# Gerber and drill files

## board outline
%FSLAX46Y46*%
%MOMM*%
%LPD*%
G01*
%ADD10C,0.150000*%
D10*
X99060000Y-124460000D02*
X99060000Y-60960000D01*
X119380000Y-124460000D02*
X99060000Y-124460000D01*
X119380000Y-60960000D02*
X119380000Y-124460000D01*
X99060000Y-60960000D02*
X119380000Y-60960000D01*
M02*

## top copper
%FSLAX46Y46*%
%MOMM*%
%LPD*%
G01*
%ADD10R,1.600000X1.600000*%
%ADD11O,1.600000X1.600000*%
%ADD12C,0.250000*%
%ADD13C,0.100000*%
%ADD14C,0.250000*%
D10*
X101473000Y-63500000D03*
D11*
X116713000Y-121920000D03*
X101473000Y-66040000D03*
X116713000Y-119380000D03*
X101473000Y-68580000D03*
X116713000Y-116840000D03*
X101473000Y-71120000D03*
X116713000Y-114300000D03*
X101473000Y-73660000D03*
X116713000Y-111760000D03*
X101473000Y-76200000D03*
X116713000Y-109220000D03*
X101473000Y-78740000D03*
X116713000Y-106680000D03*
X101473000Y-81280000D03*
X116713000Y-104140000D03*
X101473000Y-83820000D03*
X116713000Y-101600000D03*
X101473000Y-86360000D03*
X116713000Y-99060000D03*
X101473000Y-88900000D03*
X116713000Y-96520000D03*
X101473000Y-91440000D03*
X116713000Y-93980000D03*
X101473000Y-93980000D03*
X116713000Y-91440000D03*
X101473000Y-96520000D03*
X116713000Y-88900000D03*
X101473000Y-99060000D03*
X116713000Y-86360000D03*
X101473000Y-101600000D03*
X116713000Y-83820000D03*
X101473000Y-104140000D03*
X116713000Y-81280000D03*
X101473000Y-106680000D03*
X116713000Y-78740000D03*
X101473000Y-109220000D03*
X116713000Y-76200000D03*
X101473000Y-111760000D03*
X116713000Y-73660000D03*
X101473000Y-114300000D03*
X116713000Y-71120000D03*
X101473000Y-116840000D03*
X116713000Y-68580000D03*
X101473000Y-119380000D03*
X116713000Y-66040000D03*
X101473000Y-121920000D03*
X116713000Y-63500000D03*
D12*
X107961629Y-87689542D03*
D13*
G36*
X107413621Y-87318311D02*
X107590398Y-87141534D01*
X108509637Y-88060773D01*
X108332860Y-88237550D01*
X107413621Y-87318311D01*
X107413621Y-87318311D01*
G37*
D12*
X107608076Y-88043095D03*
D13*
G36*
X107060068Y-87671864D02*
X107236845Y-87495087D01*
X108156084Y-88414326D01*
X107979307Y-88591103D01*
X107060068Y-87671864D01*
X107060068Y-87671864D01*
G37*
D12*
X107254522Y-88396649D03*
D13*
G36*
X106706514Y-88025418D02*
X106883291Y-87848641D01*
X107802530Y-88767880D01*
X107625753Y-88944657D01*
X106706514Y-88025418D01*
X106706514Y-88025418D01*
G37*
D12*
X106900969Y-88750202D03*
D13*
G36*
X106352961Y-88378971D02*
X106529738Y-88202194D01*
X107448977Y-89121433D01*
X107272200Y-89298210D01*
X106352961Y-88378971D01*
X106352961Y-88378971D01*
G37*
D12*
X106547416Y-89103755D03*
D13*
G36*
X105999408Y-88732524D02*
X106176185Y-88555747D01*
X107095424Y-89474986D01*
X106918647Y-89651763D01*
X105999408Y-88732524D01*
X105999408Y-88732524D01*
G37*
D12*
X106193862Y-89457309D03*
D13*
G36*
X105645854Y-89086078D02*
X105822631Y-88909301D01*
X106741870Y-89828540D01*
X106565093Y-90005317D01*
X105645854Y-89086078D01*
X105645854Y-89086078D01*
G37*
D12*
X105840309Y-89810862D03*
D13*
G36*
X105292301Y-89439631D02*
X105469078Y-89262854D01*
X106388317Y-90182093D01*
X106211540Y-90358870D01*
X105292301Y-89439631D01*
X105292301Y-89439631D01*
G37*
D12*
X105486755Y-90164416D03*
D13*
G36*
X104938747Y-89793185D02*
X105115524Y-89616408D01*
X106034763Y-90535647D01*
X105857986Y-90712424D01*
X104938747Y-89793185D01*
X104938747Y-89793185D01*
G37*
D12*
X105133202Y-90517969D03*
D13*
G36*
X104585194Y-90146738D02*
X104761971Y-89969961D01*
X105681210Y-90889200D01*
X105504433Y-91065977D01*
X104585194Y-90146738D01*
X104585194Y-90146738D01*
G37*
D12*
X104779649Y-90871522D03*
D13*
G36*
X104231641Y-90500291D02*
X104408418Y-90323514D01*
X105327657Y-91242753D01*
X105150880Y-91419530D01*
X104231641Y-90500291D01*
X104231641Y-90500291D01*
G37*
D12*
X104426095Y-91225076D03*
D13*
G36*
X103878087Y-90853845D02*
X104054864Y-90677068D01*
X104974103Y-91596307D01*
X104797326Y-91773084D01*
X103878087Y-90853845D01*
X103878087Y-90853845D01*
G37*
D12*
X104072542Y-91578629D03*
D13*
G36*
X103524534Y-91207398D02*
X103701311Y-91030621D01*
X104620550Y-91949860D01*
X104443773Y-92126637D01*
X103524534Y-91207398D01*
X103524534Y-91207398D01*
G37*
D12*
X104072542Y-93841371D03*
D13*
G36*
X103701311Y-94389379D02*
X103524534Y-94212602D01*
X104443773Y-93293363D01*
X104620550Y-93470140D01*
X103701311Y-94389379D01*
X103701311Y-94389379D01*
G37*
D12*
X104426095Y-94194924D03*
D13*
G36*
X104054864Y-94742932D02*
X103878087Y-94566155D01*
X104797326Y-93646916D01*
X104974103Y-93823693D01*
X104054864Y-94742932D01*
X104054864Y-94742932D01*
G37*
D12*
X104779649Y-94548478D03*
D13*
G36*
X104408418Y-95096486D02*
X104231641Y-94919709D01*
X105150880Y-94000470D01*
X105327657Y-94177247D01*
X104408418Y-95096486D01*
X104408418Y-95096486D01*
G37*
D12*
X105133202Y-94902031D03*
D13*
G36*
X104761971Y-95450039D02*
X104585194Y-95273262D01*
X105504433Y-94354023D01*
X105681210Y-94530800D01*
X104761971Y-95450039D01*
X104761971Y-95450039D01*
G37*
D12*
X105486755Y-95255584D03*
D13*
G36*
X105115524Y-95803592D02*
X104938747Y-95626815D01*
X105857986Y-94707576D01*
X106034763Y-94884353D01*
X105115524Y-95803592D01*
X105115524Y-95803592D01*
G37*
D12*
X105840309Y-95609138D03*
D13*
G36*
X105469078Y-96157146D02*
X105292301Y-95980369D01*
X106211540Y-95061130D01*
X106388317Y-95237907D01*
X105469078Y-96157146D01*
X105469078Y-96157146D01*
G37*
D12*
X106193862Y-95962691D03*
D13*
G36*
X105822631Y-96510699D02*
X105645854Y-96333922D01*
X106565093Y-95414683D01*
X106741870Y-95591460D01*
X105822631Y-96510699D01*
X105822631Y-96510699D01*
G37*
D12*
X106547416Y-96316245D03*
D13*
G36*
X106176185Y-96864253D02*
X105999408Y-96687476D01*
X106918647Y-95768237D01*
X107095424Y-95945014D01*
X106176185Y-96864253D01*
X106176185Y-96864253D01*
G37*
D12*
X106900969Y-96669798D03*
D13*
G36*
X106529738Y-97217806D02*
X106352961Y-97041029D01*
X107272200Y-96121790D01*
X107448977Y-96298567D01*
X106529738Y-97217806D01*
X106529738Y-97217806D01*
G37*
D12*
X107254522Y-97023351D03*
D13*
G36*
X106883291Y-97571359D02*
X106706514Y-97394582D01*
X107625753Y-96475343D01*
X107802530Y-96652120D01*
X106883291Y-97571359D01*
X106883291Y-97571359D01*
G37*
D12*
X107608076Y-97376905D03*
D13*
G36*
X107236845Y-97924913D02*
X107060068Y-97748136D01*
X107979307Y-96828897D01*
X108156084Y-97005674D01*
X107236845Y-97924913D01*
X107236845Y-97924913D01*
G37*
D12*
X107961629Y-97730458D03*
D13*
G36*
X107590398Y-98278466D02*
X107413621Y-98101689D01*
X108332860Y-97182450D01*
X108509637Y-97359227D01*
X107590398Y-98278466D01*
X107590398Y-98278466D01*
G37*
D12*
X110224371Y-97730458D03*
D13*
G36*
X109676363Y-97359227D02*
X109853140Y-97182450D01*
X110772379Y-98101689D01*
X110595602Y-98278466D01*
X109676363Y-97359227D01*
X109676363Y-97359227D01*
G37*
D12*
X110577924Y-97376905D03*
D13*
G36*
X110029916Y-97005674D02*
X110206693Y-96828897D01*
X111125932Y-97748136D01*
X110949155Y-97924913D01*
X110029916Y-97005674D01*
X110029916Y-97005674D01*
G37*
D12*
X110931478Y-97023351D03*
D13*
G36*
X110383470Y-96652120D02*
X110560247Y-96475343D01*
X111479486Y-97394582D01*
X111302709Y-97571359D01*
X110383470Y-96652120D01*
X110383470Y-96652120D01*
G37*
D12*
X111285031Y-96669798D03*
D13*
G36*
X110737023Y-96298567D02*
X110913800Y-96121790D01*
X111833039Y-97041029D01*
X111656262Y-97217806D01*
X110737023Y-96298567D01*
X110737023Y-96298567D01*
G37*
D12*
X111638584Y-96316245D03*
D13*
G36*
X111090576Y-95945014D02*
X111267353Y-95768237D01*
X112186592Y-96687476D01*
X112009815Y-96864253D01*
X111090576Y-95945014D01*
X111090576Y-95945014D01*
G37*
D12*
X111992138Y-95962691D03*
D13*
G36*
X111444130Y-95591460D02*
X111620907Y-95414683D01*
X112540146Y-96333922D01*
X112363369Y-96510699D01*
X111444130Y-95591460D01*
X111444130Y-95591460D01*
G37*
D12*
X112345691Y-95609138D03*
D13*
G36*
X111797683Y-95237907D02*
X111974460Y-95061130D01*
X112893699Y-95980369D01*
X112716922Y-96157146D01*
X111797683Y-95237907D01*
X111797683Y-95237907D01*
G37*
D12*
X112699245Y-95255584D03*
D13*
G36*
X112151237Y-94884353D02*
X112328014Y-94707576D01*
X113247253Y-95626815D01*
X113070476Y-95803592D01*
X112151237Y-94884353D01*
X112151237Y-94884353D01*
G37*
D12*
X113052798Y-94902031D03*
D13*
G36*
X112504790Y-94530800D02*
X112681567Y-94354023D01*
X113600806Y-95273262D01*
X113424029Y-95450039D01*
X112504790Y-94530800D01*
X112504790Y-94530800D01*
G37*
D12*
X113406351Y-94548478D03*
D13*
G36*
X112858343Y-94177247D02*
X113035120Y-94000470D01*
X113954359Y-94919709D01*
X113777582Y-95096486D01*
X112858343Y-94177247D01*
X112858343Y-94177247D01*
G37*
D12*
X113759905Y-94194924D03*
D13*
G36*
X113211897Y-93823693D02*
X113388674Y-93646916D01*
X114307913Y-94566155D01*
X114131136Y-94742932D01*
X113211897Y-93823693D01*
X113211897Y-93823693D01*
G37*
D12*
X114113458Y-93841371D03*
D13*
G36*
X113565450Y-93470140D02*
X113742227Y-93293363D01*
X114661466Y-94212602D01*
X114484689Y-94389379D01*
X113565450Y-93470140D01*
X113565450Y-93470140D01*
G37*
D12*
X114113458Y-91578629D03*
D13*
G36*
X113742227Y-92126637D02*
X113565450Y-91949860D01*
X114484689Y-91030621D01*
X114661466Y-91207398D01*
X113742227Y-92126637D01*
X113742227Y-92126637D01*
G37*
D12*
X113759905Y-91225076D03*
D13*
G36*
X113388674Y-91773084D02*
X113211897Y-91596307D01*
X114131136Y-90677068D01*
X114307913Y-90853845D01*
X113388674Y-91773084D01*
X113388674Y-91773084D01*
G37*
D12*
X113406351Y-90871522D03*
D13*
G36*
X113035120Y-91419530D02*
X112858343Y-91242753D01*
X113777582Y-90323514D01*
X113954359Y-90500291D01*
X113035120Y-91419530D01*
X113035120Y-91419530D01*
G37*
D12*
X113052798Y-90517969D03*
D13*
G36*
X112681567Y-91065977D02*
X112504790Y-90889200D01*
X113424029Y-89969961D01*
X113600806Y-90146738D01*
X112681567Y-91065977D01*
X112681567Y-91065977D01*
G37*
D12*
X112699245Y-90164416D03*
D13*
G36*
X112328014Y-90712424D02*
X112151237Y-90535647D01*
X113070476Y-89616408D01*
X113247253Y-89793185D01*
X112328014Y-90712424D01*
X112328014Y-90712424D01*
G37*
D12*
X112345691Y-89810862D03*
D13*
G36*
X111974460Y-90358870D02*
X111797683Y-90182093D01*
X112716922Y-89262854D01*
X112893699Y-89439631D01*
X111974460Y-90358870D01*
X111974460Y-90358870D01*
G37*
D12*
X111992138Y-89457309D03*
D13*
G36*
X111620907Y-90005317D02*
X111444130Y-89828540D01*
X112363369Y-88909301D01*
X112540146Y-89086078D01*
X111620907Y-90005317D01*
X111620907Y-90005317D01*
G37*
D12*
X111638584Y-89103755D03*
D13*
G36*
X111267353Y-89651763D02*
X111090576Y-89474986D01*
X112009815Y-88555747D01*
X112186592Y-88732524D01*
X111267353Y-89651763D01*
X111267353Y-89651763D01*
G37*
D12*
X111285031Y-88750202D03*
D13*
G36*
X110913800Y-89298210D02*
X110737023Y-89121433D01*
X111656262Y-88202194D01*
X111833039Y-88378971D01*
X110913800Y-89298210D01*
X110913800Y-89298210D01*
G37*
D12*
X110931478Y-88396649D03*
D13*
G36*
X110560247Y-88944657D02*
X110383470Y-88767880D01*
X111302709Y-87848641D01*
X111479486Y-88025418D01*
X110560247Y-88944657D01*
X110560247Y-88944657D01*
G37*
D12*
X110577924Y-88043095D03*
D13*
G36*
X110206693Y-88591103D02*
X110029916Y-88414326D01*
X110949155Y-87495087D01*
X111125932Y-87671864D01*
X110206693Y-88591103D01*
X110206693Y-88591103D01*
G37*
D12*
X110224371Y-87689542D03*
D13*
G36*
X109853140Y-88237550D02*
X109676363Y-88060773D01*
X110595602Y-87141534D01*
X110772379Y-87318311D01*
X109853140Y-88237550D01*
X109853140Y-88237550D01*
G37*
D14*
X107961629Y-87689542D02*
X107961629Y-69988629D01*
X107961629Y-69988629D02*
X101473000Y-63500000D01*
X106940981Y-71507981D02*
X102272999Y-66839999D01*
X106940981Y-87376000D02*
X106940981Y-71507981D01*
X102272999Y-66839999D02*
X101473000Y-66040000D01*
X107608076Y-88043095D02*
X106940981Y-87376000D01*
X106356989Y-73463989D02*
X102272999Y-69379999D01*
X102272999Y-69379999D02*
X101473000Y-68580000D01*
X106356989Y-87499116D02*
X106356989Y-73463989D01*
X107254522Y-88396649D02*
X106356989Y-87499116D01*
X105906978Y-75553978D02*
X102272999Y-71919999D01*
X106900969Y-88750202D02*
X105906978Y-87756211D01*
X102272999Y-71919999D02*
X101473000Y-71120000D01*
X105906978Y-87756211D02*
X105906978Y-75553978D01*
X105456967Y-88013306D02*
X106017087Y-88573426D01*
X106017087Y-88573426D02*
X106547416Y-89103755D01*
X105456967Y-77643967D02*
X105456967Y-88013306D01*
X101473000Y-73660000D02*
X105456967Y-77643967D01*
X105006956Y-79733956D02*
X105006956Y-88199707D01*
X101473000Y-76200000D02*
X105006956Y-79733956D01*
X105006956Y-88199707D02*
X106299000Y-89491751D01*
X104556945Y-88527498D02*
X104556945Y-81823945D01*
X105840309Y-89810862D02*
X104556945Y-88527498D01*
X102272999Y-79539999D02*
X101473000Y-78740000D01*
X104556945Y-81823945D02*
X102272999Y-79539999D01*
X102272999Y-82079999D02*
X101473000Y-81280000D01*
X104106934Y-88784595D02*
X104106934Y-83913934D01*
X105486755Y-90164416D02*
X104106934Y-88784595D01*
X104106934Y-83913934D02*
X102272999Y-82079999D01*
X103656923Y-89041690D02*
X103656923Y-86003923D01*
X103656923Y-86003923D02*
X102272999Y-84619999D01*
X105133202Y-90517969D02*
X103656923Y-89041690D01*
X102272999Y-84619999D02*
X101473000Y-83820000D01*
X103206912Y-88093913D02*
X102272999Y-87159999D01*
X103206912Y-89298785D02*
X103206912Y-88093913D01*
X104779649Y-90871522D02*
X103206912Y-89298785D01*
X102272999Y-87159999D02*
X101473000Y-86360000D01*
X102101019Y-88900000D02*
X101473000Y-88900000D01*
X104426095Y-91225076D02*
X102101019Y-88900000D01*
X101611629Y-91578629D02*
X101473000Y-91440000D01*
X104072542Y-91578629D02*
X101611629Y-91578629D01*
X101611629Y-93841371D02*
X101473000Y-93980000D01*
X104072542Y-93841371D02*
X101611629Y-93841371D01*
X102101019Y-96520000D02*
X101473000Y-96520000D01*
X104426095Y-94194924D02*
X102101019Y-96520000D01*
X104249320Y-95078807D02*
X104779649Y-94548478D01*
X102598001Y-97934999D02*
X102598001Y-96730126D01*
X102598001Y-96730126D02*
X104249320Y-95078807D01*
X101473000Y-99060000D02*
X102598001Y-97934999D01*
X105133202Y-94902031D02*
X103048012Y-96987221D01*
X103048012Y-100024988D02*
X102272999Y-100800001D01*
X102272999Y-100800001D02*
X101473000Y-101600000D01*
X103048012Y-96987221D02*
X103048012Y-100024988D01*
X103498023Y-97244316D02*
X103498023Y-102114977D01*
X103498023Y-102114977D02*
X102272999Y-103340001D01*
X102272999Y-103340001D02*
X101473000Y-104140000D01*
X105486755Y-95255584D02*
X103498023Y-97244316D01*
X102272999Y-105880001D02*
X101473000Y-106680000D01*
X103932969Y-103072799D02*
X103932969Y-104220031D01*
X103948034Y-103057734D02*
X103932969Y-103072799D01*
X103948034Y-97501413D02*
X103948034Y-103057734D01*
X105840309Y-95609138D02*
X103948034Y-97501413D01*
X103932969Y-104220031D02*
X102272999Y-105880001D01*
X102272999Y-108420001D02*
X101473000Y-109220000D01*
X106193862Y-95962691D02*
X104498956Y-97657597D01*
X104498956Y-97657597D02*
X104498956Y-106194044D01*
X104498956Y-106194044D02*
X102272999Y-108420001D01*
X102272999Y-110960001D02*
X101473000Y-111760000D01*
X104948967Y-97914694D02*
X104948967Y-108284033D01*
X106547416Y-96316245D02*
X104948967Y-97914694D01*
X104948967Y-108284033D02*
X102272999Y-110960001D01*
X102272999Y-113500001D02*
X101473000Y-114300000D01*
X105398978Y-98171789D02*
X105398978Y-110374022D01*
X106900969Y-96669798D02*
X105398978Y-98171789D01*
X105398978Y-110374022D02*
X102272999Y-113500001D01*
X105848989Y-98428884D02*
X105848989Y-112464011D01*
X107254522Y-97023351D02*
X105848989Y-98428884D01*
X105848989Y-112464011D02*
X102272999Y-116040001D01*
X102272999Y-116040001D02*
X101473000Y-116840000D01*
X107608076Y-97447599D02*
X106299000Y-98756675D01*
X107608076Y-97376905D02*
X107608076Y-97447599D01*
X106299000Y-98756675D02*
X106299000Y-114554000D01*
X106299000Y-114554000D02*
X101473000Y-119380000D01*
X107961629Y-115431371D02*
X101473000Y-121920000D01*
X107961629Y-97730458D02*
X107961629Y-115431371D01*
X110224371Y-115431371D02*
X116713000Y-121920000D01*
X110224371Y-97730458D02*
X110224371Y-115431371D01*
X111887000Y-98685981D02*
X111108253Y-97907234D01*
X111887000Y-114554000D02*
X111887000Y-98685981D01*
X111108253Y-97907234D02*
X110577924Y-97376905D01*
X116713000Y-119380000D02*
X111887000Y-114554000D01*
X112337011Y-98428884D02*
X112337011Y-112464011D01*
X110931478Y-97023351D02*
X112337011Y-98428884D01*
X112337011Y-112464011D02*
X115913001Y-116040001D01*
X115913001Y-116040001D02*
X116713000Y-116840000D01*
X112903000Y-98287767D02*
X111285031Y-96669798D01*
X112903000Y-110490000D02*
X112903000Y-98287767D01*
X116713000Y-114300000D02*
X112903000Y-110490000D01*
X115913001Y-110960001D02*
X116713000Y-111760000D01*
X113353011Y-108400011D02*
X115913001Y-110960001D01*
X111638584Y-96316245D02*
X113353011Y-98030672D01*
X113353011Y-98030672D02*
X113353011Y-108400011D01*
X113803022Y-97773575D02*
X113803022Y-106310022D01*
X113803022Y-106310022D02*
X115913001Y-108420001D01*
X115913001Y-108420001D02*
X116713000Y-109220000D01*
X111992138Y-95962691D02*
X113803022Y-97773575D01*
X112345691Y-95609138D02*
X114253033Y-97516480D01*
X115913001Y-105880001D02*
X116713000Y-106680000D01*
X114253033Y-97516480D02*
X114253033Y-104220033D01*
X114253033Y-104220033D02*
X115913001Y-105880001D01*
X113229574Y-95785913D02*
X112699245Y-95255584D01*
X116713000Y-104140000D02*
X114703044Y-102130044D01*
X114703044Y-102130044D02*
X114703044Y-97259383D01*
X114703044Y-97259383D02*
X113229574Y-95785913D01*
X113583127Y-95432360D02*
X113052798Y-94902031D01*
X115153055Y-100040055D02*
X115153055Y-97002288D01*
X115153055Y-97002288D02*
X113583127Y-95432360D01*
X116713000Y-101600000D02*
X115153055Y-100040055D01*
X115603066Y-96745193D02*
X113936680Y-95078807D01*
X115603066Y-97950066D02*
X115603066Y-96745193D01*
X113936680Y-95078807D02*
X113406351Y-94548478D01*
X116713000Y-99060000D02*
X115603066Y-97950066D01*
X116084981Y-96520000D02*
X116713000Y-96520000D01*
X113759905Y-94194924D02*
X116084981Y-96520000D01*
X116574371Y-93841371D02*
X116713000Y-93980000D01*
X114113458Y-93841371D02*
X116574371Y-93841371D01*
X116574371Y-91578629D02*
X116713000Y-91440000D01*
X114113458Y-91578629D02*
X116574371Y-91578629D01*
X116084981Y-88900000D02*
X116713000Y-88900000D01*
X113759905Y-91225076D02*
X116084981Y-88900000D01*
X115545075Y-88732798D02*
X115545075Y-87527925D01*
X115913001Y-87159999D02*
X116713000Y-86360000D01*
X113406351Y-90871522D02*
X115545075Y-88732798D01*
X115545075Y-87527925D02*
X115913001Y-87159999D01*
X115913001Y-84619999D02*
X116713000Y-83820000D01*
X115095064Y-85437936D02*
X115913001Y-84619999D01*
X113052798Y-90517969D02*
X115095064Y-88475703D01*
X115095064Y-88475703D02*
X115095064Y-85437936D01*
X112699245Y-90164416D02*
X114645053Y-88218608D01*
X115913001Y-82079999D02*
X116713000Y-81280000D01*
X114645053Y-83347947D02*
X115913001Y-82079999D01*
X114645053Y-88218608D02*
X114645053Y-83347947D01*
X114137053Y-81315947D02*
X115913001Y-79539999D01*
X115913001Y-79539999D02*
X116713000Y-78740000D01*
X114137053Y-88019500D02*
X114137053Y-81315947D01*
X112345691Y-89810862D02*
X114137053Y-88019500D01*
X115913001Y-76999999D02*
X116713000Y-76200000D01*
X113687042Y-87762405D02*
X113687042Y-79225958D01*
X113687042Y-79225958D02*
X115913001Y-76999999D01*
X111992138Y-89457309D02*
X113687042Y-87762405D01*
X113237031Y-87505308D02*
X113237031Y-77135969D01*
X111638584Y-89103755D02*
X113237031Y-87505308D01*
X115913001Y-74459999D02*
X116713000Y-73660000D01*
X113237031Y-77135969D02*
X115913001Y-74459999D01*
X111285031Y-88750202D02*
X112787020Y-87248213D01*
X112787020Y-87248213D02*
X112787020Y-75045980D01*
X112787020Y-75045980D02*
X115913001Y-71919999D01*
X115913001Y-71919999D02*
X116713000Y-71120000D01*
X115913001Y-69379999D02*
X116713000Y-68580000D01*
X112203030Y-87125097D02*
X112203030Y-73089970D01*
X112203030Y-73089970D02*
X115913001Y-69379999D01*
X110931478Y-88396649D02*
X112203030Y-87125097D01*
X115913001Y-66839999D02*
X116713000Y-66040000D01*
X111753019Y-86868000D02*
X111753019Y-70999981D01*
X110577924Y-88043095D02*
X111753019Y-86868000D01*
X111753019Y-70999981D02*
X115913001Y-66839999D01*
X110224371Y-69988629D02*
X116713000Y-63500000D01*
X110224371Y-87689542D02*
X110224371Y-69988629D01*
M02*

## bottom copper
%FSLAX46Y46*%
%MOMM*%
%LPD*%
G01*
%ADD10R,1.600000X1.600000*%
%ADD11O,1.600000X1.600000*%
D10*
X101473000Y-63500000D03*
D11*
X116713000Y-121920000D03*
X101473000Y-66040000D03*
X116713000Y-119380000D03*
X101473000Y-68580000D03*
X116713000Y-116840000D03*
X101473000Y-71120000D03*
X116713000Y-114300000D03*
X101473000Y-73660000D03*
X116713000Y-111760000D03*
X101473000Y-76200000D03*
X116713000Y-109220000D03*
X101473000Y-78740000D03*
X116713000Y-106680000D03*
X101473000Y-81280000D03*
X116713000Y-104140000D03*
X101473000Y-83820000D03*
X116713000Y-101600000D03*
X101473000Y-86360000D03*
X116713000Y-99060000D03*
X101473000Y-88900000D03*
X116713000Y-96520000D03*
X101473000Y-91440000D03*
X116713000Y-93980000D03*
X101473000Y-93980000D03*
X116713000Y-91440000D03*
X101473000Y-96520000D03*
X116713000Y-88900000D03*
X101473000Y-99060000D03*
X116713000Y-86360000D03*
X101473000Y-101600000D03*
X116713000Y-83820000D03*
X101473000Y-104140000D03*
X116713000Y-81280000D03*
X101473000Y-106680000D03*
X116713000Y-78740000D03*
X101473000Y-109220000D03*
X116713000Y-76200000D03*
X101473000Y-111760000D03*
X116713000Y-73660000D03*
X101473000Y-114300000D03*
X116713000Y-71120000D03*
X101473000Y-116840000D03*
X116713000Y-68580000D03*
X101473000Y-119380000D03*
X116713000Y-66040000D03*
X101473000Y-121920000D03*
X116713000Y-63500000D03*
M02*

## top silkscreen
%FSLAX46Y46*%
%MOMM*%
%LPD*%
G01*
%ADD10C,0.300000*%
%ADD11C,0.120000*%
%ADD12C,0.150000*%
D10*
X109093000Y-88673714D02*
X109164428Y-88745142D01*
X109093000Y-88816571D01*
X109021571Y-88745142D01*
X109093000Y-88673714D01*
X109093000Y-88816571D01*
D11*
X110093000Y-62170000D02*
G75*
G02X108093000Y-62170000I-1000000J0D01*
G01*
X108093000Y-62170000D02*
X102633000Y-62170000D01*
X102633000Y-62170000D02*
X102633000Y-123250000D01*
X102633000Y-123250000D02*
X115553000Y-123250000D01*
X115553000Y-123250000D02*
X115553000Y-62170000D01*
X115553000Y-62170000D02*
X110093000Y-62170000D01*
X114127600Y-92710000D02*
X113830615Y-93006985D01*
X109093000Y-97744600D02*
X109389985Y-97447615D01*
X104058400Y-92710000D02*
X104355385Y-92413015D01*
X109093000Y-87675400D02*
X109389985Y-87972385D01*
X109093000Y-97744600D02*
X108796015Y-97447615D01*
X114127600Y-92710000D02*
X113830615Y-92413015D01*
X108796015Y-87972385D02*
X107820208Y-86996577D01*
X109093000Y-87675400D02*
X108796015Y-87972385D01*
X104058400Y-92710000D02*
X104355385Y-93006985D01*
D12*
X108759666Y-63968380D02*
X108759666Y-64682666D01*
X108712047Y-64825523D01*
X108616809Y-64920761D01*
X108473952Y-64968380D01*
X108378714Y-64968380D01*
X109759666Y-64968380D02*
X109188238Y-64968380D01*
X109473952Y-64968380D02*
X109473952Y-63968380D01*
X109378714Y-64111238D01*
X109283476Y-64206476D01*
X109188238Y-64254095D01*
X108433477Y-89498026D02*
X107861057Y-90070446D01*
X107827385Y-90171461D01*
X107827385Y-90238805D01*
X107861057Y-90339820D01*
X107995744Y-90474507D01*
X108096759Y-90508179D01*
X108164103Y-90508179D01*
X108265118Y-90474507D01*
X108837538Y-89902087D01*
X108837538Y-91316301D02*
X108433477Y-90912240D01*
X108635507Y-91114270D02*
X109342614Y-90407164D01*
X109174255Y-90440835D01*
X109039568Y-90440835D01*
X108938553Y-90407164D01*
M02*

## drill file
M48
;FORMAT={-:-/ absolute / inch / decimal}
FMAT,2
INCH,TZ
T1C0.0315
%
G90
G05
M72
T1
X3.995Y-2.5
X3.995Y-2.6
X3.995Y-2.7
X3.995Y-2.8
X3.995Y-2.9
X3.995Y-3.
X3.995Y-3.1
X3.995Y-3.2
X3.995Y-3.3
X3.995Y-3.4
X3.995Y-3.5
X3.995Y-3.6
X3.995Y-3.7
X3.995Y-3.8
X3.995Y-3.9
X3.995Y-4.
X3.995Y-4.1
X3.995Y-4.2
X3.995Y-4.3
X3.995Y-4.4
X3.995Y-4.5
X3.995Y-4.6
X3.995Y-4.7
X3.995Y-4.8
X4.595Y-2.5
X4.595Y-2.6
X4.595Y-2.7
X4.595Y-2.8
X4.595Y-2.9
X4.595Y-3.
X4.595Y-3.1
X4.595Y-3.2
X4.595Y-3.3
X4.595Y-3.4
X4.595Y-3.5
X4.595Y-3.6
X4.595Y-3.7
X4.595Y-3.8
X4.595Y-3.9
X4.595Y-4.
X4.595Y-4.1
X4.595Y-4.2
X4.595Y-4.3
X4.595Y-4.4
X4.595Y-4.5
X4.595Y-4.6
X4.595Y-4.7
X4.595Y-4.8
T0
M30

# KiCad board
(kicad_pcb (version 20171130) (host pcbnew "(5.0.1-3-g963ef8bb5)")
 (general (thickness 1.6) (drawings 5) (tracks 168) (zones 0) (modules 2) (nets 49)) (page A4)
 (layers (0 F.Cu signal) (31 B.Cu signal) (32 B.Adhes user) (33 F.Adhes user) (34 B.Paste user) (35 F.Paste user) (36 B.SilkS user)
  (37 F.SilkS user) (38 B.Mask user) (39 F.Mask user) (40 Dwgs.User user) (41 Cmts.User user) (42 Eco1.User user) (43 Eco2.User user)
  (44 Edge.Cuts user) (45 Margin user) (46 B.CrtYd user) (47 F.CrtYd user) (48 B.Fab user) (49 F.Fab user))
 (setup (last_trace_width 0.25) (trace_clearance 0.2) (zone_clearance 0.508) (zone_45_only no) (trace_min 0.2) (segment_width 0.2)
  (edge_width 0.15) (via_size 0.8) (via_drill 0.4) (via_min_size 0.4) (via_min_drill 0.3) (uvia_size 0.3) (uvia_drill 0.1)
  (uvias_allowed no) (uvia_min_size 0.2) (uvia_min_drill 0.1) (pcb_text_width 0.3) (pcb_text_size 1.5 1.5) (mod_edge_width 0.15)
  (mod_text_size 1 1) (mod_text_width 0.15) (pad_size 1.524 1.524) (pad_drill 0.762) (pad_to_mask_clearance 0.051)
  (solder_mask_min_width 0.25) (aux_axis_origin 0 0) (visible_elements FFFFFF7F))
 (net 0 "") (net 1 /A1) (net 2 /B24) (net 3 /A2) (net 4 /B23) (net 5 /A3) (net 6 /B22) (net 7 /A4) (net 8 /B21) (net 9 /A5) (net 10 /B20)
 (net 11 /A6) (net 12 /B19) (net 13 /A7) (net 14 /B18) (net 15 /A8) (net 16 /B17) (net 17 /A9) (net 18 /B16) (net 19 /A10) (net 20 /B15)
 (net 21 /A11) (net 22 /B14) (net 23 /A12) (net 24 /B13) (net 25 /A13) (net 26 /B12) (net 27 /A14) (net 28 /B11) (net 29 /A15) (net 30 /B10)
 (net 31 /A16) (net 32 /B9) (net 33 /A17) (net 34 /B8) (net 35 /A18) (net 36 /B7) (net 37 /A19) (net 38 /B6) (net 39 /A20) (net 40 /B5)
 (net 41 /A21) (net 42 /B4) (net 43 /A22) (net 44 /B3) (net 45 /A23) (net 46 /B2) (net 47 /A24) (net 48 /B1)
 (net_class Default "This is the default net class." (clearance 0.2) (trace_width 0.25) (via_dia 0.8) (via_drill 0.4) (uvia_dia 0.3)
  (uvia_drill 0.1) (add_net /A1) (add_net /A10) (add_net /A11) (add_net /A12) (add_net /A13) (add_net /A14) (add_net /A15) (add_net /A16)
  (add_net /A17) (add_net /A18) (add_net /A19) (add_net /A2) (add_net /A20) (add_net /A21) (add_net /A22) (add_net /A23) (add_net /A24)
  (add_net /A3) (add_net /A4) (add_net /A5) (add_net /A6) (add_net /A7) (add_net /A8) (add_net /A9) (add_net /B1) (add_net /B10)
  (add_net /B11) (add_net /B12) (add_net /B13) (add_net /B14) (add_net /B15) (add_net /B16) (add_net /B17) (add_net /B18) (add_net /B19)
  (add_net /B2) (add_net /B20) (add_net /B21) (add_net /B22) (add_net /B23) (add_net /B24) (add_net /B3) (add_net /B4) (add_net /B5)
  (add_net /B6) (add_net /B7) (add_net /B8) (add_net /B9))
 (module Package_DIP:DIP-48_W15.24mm (layer F.Cu) (at 101.473 63.5)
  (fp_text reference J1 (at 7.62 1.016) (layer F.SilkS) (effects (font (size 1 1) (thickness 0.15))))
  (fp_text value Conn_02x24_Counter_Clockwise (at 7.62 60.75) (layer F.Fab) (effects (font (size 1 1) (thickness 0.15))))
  (fp_arc (start 7.62 -1.33) (end 6.62 -1.33) (angle -180) (layer F.SilkS) (width 0.12))
  (fp_line (start 6.62 -1.33) (end 1.16 -1.33) (layer F.SilkS) (width 0.12))
  (fp_line (start 1.16 -1.33) (end 1.16 59.75) (layer F.SilkS) (width 0.12))
  (fp_line (start 1.16 59.75) (end 14.08 59.75) (layer F.SilkS) (width 0.12))
  (fp_line (start 14.08 59.75) (end 14.08 -1.33) (layer F.SilkS) (width 0.12))
  (fp_line (start 14.08 -1.33) (end 8.62 -1.33) (layer F.SilkS) (width 0.12))
  (pad 1 thru_hole rect (at 0 0) (size 1.6 1.6) (drill 0.8) (layers *.Cu *.Mask) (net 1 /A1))
  (pad 25 thru_hole oval (at 15.24 58.42) (size 1.6 1.6) (drill 0.8) (layers *.Cu *.Mask) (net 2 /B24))
  (pad 2 thru_hole oval (at 0 2.54) (size 1.6 1.6) (drill 0.8) (layers *.Cu *.Mask) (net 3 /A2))
  (pad 26 thru_hole oval (at 15.24 55.88) (size 1.6 1.6) (drill 0.8) (layers *.Cu *.Mask) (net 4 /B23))
  (pad 3 thru_hole oval (at 0 5.08) (size 1.6 1.6) (drill 0.8) (layers *.Cu *.Mask) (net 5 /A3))
  (pad 27 thru_hole oval (at 15.24 53.34) (size 1.6 1.6) (drill 0.8) (layers *.Cu *.Mask) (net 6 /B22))
  (pad 4 thru_hole oval (at 0 7.62) (size 1.6 1.6) (drill 0.8) (layers *.Cu *.Mask) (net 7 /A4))
  (pad 28 thru_hole oval (at 15.24 50.8) (size 1.6 1.6) (drill 0.8) (layers *.Cu *.Mask) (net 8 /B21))
  (pad 5 thru_hole oval (at 0 10.16) (size 1.6 1.6) (drill 0.8) (layers *.Cu *.Mask) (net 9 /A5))
  (pad 29 thru_hole oval (at 15.24 48.26) (size 1.6 1.6) (drill 0.8) (layers *.Cu *.Mask) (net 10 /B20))
  (pad 6 thru_hole oval (at 0 12.7) (size 1.6 1.6) (drill 0.8) (layers *.Cu *.Mask) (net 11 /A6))
  (pad 30 thru_hole oval (at 15.24 45.72) (size 1.6 1.6) (drill 0.8) (layers *.Cu *.Mask) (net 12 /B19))
  (pad 7 thru_hole oval (at 0 15.24) (size 1.6 1.6) (drill 0.8) (layers *.Cu *.Mask) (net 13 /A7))
  (pad 31 thru_hole oval (at 15.24 43.18) (size 1.6 1.6) (drill 0.8) (layers *.Cu *.Mask) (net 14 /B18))
  (pad 8 thru_hole oval (at 0 17.78) (size 1.6 1.6) (drill 0.8) (layers *.Cu *.Mask) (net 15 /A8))
  (pad 32 thru_hole oval (at 15.24 40.64) (size 1.6 1.6) (drill 0.8) (layers *.Cu *.Mask) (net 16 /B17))
  (pad 9 thru_hole oval (at 0 20.32) (size 1.6 1.6) (drill 0.8) (layers *.Cu *.Mask) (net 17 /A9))
  (pad 33 thru_hole oval (at 15.24 38.1) (size 1.6 1.6) (drill 0.8) (layers *.Cu *.Mask) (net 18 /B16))
  (pad 10 thru_hole oval (at 0 22.86) (size 1.6 1.6) (drill 0.8) (layers *.Cu *.Mask) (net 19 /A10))
  (pad 34 thru_hole oval (at 15.24 35.56) (size 1.6 1.6) (drill 0.8) (layers *.Cu *.Mask) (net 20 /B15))
  (pad 11 thru_hole oval (at 0 25.4) (size 1.6 1.6) (drill 0.8) (layers *.Cu *.Mask) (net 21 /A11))
  (pad 35 thru_hole oval (at 15.24 33.02) (size 1.6 1.6) (drill 0.8) (layers *.Cu *.Mask) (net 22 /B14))
  (pad 12 thru_hole oval (at 0 27.94) (size 1.6 1.6) (drill 0.8) (layers *.Cu *.Mask) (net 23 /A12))
  (pad 36 thru_hole oval (at 15.24 30.48) (size 1.6 1.6) (drill 0.8) (layers *.Cu *.Mask) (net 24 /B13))
  (pad 13 thru_hole oval (at 0 30.48) (size 1.6 1.6) (drill 0.8) (layers *.Cu *.Mask) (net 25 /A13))
  (pad 37 thru_hole oval (at 15.24 27.94) (size 1.6 1.6) (drill 0.8) (layers *.Cu *.Mask) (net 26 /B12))
  (pad 14 thru_hole oval (at 0 33.02) (size 1.6 1.6) (drill 0.8) (layers *.Cu *.Mask) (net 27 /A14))
  (pad 38 thru_hole oval (at 15.24 25.4) (size 1.6 1.6) (drill 0.8) (layers *.Cu *.Mask) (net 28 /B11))
  (pad 15 thru_hole oval (at 0 35.56) (size 1.6 1.6) (drill 0.8) (layers *.Cu *.Mask) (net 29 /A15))
  (pad 39 thru_hole oval (at 15.24 22.86) (size 1.6 1.6) (drill 0.8) (layers *.Cu *.Mask) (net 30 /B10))
  (pad 16 thru_hole oval (at 0 38.1) (size 1.6 1.6) (drill 0.8) (layers *.Cu *.Mask) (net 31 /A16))
  (pad 40 thru_hole oval (at 15.24 20.32) (size 1.6 1.6) (drill 0.8) (layers *.Cu *.Mask) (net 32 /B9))
  (pad 17 thru_hole oval (at 0 40.64) (size 1.6 1.6) (drill 0.8) (layers *.Cu *.Mask) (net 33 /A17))
  (pad 41 thru_hole oval (at 15.24 17.78) (size 1.6 1.6) (drill 0.8) (layers *.Cu *.Mask) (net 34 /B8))
  (pad 18 thru_hole oval (at 0 43.18) (size 1.6 1.6) (drill 0.8) (layers *.Cu *.Mask) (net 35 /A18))
  (pad 42 thru_hole oval (at 15.24 15.24) (size 1.6 1.6) (drill 0.8) (layers *.Cu *.Mask) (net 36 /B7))
  (pad 19 thru_hole oval (at 0 45.72) (size 1.6 1.6) (drill 0.8) (layers *.Cu *.Mask) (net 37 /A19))
  (pad 43 thru_hole oval (at 15.24 12.7) (size 1.6 1.6) (drill 0.8) (layers *.Cu *.Mask) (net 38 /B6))
  (pad 20 thru_hole oval (at 0 48.26) (size 1.6 1.6) (drill 0.8) (layers *.Cu *.Mask) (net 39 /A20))
  (pad 44 thru_hole oval (at 15.24 10.16) (size 1.6 1.6) (drill 0.8) (layers *.Cu *.Mask) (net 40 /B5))
  (pad 21 thru_hole oval (at 0 50.8) (size 1.6 1.6) (drill 0.8) (layers *.Cu *.Mask) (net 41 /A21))
  (pad 45 thru_hole oval (at 15.24 7.62) (size 1.6 1.6) (drill 0.8) (layers *.Cu *.Mask) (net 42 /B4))
  (pad 22 thru_hole oval (at 0 53.34) (size 1.6 1.6) (drill 0.8) (layers *.Cu *.Mask) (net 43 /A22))
  (pad 46 thru_hole oval (at 15.24 5.08) (size 1.6 1.6) (drill 0.8) (layers *.Cu *.Mask) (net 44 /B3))
  (pad 23 thru_hole oval (at 0 55.88) (size 1.6 1.6) (drill 0.8) (layers *.Cu *.Mask) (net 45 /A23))
  (pad 47 thru_hole oval (at 15.24 2.54) (size 1.6 1.6) (drill 0.8) (layers *.Cu *.Mask) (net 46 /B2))
  (pad 24 thru_hole oval (at 0 58.42) (size 1.6 1.6) (drill 0.8) (layers *.Cu *.Mask) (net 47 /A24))
  (pad 48 thru_hole oval (at 15.24 0) (size 1.6 1.6) (drill 0.8) (layers *.Cu *.Mask) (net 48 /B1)))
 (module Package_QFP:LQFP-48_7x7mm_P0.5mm (layer F.Cu) (at 109.093 92.71 315)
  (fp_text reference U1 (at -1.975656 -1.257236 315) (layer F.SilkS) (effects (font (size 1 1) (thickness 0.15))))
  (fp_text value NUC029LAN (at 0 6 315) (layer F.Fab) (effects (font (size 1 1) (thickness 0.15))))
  (fp_line (start 3.56 -3.56) (end 3.56 -3.14) (layer F.SilkS) (width 0.12))
  (fp_line (start 3.56 3.56) (end 3.56 3.14) (layer F.SilkS) (width 0.12))
  (fp_line (start -3.56 3.56) (end -3.56 3.14) (layer F.SilkS) (width 0.12))
  (fp_line (start -3.56 -3.56) (end -3.14 -3.56) (layer F.SilkS) (width 0.12))
  (fp_line (start 3.56 3.56) (end 3.14 3.56) (layer F.SilkS) (width 0.12))
  (fp_line (start 3.56 -3.56) (end 3.14 -3.56) (layer F.SilkS) (width 0.12))
  (fp_line (start -3.56 -3.14) (end -4.94 -3.14) (layer F.SilkS) (width 0.12))
  (fp_line (start -3.56 -3.56) (end -3.56 -3.14) (layer F.SilkS) (width 0.12))
  (fp_line (start -3.56 3.56) (end -3.14 3.56) (layer F.SilkS) (width 0.12))
  (pad 1 smd rect (at -4.35 -2.75 315) (size 1.3 0.25) (layers F.Cu F.Paste F.Mask) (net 1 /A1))
  (pad 2 smd rect (at -4.35 -2.25 315) (size 1.3 0.25) (layers F.Cu F.Paste F.Mask) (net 3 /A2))
  (pad 3 smd rect (at -4.35 -1.749999 315) (size 1.3 0.25) (layers F.Cu F.Paste F.Mask) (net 5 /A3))
  (pad 4 smd rect (at -4.35 -1.25 315) (size 1.3 0.25) (layers F.Cu F.Paste F.Mask) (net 7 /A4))
  (pad 5 smd rect (at -4.35 -0.750001 315) (size 1.3 0.25) (layers F.Cu F.Paste F.Mask) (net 9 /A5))
  (pad 6 smd rect (at -4.35 -0.25 315) (size 1.3 0.25) (layers F.Cu F.Paste F.Mask) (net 11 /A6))
  (pad 7 smd rect (at -4.35 0.25 315) (size 1.3 0.25) (layers F.Cu F.Paste F.Mask) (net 13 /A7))
  (pad 8 smd rect (at -4.35 0.750001 315) (size 1.3 0.25) (layers F.Cu F.Paste F.Mask) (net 15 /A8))
  (pad 9 smd rect (at -4.35 1.25 315) (size 1.3 0.25) (layers F.Cu F.Paste F.Mask) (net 17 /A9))
  (pad 10 smd rect (at -4.35 1.749999 315) (size 1.3 0.25) (layers F.Cu F.Paste F.Mask) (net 19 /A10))
  (pad 11 smd rect (at -4.35 2.25 315) (size 1.3 0.25) (layers F.Cu F.Paste F.Mask) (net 21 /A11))
  (pad 12 smd rect (at -4.35 2.75 315) (size 1.3 0.25) (layers F.Cu F.Paste F.Mask) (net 23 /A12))
  (pad 13 smd rect (at -2.75 4.35 45) (size 1.3 0.25) (layers F.Cu F.Paste F.Mask) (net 25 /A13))
  (pad 14 smd rect (at -2.25 4.35 45) (size 1.3 0.25) (layers F.Cu F.Paste F.Mask) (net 27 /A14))
  (pad 15 smd rect (at -1.749999 4.35 45) (size 1.3 0.25) (layers F.Cu F.Paste F.Mask) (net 29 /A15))
  (pad 16 smd rect (at -1.25 4.35 45) (size 1.3 0.25) (layers F.Cu F.Paste F.Mask) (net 31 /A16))
  (pad 17 smd rect (at -0.750001 4.35 45) (size 1.3 0.25) (layers F.Cu F.Paste F.Mask) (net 33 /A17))
  (pad 18 smd rect (at -0.25 4.35 45) (size 1.3 0.25) (layers F.Cu F.Paste F.Mask) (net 35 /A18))
  (pad 19 smd rect (at 0.25 4.35 45) (size 1.3 0.25) (layers F.Cu F.Paste F.Mask) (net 37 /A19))
  (pad 20 smd rect (at 0.750001 4.35 45) (size 1.3 0.25) (layers F.Cu F.Paste F.Mask) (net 39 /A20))
  (pad 21 smd rect (at 1.25 4.35 45) (size 1.3 0.25) (layers F.Cu F.Paste F.Mask) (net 41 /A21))
  (pad 22 smd rect (at 1.749999 4.35 45) (size 1.3 0.25) (layers F.Cu F.Paste F.Mask) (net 43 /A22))
  (pad 23 smd rect (at 2.25 4.35 45) (size 1.3 0.25) (layers F.Cu F.Paste F.Mask) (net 45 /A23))
  (pad 24 smd rect (at 2.75 4.35 45) (size 1.3 0.25) (layers F.Cu F.Paste F.Mask) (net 47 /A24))
  (pad 25 smd rect (at 4.35 2.75 315) (size 1.3 0.25) (layers F.Cu F.Paste F.Mask) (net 2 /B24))
  (pad 26 smd rect (at 4.35 2.25 315) (size 1.3 0.25) (layers F.Cu F.Paste F.Mask) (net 4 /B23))
  (pad 27 smd rect (at 4.35 1.749999 315) (size 1.3 0.25) (layers F.Cu F.Paste F.Mask) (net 6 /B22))
  (pad 28 smd rect (at 4.35 1.25 315) (size 1.3 0.25) (layers F.Cu F.Paste F.Mask) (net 8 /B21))
  (pad 29 smd rect (at 4.35 0.750001 315) (size 1.3 0.25) (layers F.Cu F.Paste F.Mask) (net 10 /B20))
  (pad 30 smd rect (at 4.35 0.25 315) (size 1.3 0.25) (layers F.Cu F.Paste F.Mask) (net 12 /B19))
  (pad 31 smd rect (at 4.35 -0.25 315) (size 1.3 0.25) (layers F.Cu F.Paste F.Mask) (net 14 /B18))
  (pad 32 smd rect (at 4.35 -0.750001 315) (size 1.3 0.25) (layers F.Cu F.Paste F.Mask) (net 16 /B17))
  (pad 33 smd rect (at 4.35 -1.25 315) (size 1.3 0.25) (layers F.Cu F.Paste F.Mask) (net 18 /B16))
  (pad 34 smd rect (at 4.35 -1.749999 315) (size 1.3 0.25) (layers F.Cu F.Paste F.Mask) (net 20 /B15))
  (pad 35 smd rect (at 4.35 -2.25 315) (size 1.3 0.25) (layers F.Cu F.Paste F.Mask) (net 22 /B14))
  (pad 36 smd rect (at 4.35 -2.75 315) (size 1.3 0.25) (layers F.Cu F.Paste F.Mask) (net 24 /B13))
  (pad 37 smd rect (at 2.75 -4.35 45) (size 1.3 0.25) (layers F.Cu F.Paste F.Mask) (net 26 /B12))
  (pad 38 smd rect (at 2.25 -4.35 45) (size 1.3 0.25) (layers F.Cu F.Paste F.Mask) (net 28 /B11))
  (pad 39 smd rect (at 1.749999 -4.35 45) (size 1.3 0.25) (layers F.Cu F.Paste F.Mask) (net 30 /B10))
  (pad 40 smd rect (at 1.25 -4.35 45) (size 1.3 0.25) (layers F.Cu F.Paste F.Mask) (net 32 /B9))
  (pad 41 smd rect (at 0.750001 -4.35 45) (size 1.3 0.25) (layers F.Cu F.Paste F.Mask) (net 34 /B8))
  (pad 42 smd rect (at 0.25 -4.35 45) (size 1.3 0.25) (layers F.Cu F.Paste F.Mask) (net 36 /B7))
  (pad 43 smd rect (at -0.25 -4.35 45) (size 1.3 0.25) (layers F.Cu F.Paste F.Mask) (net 38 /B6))
  (pad 44 smd rect (at -0.750001 -4.35 45) (size 1.3 0.25) (layers F.Cu F.Paste F.Mask) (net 40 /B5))
  (pad 45 smd rect (at -1.25 -4.35 45) (size 1.3 0.25) (layers F.Cu F.Paste F.Mask) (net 42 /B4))
  (pad 46 smd rect (at -1.749999 -4.35 45) (size 1.3 0.25) (layers F.Cu F.Paste F.Mask) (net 44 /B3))
  (pad 47 smd rect (at -2.25 -4.35 45) (size 1.3 0.25) (layers F.Cu F.Paste F.Mask) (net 46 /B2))
  (pad 48 smd rect (at -2.75 -4.35 45) (size 1.3 0.25) (layers F.Cu F.Paste F.Mask) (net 48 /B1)))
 (gr_line (start 99.06 124.46) (end 99.06 60.96) (layer Edge.Cuts) (width 0.15))
 (gr_line (start 119.38 124.46) (end 99.06 124.46) (layer Edge.Cuts) (width 0.15))
 (gr_line (start 119.38 60.96) (end 119.38 124.46) (layer Edge.Cuts) (width 0.15))
 (gr_line (start 99.06 60.96) (end 119.38 60.96) (layer Edge.Cuts) (width 0.15))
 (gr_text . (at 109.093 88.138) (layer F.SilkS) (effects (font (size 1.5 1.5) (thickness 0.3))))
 (segment (start 107.961629 87.689542) (end 107.961629 69.988629) (width 0.25) (layer F.Cu) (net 1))
 (segment (start 107.961629 69.988629) (end 101.473 63.5) (width 0.25) (layer F.Cu) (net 1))
 (segment (start 106.940981 71.507981) (end 102.272999 66.839999) (width 0.25) (layer F.Cu) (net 3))
 (segment (start 106.940981 87.376) (end 106.940981 71.507981) (width 0.25) (layer F.Cu) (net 3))
 (segment (start 102.272999 66.839999) (end 101.473 66.04) (width 0.25) (layer F.Cu) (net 3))
 (segment (start 107.608076 88.043095) (end 106.940981 87.376) (width 0.25) (layer F.Cu) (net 3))
 (segment (start 106.356989 73.463989) (end 102.272999 69.379999) (width 0.25) (layer F.Cu) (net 5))
 (segment (start 102.272999 69.379999) (end 101.473 68.58) (width 0.25) (layer F.Cu) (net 5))
 (segment (start 106.356989 87.499116) (end 106.356989 73.463989) (width 0.25) (layer F.Cu) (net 5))
 (segment (start 107.254522 88.396649) (end 106.356989 87.499116) (width 0.25) (layer F.Cu) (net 5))
 (segment (start 105.906978 75.553978) (end 102.272999 71.919999) (width 0.25) (layer F.Cu) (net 7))
 (segment (start 106.900969 88.750202) (end 105.906978 87.756211) (width 0.25) (layer F.Cu) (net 7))
 (segment (start 102.272999 71.919999) (end 101.473 71.12) (width 0.25) (layer F.Cu) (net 7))
 (segment (start 105.906978 87.756211) (end 105.906978 75.553978) (width 0.25) (layer F.Cu) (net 7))
 (segment (start 105.456967 88.013306) (end 106.017087 88.573426) (width 0.25) (layer F.Cu) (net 9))
 (segment (start 106.017087 88.573426) (end 106.547416 89.103755) (width 0.25) (layer F.Cu) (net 9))
 (segment (start 105.456967 77.643967) (end 105.456967 88.013306) (width 0.25) (layer F.Cu) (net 9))
 (segment (start 101.473 73.66) (end 105.456967 77.643967) (width 0.25) (layer F.Cu) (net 9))
 (segment (start 105.006956 79.733956) (end 105.006956 88.199707) (width 0.25) (layer F.Cu) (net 11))
 (segment (start 101.473 76.2) (end 105.006956 79.733956) (width 0.25) (layer F.Cu) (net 11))
 (segment (start 105.006956 88.199707) (end 106.299 89.491751) (width 0.25) (layer F.Cu) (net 11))
 (segment (start 104.556945 88.527498) (end 104.556945 81.823945) (width 0.25) (layer F.Cu) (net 13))
 (segment (start 105.840309 89.810862) (end 104.556945 88.527498) (width 0.25) (layer F.Cu) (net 13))
 (segment (start 102.272999 79.539999) (end 101.473 78.74) (width 0.25) (layer F.Cu) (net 13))
 (segment (start 104.556945 81.823945) (end 102.272999 79.539999) (width 0.25) (layer F.Cu) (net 13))
 (segment (start 102.272999 82.079999) (end 101.473 81.28) (width 0.25) (layer F.Cu) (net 15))
 (segment (start 104.106934 88.784595) (end 104.106934 83.913934) (width 0.25) (layer F.Cu) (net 15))
 (segment (start 105.486755 90.164416) (end 104.106934 88.784595) (width 0.25) (layer F.Cu) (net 15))
 (segment (start 104.106934 83.913934) (end 102.272999 82.079999) (width 0.25) (layer F.Cu) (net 15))
 (segment (start 103.656923 89.04169) (end 103.656923 86.003923) (width 0.25) (layer F.Cu) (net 17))
 (segment (start 103.656923 86.003923) (end 102.272999 84.619999) (width 0.25) (layer F.Cu) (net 17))
 (segment (start 105.133202 90.517969) (end 103.656923 89.04169) (width 0.25) (layer F.Cu) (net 17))
 (segment (start 102.272999 84.619999) (end 101.473 83.82) (width 0.25) (layer F.Cu) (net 17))
 (segment (start 103.206912 88.093913) (end 102.272999 87.159999) (width 0.25) (layer F.Cu) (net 19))
 (segment (start 103.206912 89.298785) (end 103.206912 88.093913) (width 0.25) (layer F.Cu) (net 19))
 (segment (start 104.779649 90.871522) (end 103.206912 89.298785) (width 0.25) (layer F.Cu) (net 19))
 (segment (start 102.272999 87.159999) (end 101.473 86.36) (width 0.25) (layer F.Cu) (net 19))
 (segment (start 102.101019 88.9) (end 101.473 88.9) (width 0.25) (layer F.Cu) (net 21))
 (segment (start 104.426095 91.225076) (end 102.101019 88.9) (width 0.25) (layer F.Cu) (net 21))
 (segment (start 101.611629 91.578629) (end 101.473 91.44) (width 0.25) (layer F.Cu) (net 23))
 (segment (start 104.072542 91.578629) (end 101.611629 91.578629) (width 0.25) (layer F.Cu) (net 23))
 (segment (start 101.611629 93.841371) (end 101.473 93.98) (width 0.25) (layer F.Cu) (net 25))
 (segment (start 104.072542 93.841371) (end 101.611629 93.841371) (width 0.25) (layer F.Cu) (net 25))
 (segment (start 102.101019 96.52) (end 101.473 96.52) (width 0.25) (layer F.Cu) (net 27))
 (segment (start 104.426095 94.194924) (end 102.101019 96.52) (width 0.25) (layer F.Cu) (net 27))
 (segment (start 104.24932 95.078807) (end 104.779649 94.548478) (width 0.25) (layer F.Cu) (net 29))
 (segment (start 102.598001 97.934999) (end 102.598001 96.730126) (width 0.25) (layer F.Cu) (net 29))
 (segment (start 102.598001 96.730126) (end 104.24932 95.078807) (width 0.25) (layer F.Cu) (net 29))
 (segment (start 101.473 99.06) (end 102.598001 97.934999) (width 0.25) (layer F.Cu) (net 29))
 (segment (start 105.133202 94.902031) (end 103.048012 96.987221) (width 0.25) (layer F.Cu) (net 31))
 (segment (start 103.048012 100.024988) (end 102.272999 100.800001) (width 0.25) (layer F.Cu) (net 31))
 (segment (start 102.272999 100.800001) (end 101.473 101.6) (width 0.25) (layer F.Cu) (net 31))
 (segment (start 103.048012 96.987221) (end 103.048012 100.024988) (width 0.25) (layer F.Cu) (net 31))
 (segment (start 103.498023 97.244316) (end 103.498023 102.114977) (width 0.25) (layer F.Cu) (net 33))
 (segment (start 103.498023 102.114977) (end 102.272999 103.340001) (width 0.25) (layer F.Cu) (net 33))
 (segment (start 102.272999 103.340001) (end 101.473 104.14) (width 0.25) (layer F.Cu) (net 33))
 (segment (start 105.486755 95.255584) (end 103.498023 97.244316) (width 0.25) (layer F.Cu) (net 33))
 (segment (start 102.272999 105.880001) (end 101.473 106.68) (width 0.25) (layer F.Cu) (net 35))
 (segment (start 103.932969 103.072799) (end 103.932969 104.220031) (width 0.25) (layer F.Cu) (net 35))
 (segment (start 103.948034 103.057734) (end 103.932969 103.072799) (width 0.25) (layer F.Cu) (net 35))
 (segment (start 103.948034 97.501413) (end 103.948034 103.057734) (width 0.25) (layer F.Cu) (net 35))
 (segment (start 105.840309 95.609138) (end 103.948034 97.501413) (width 0.25) (layer F.Cu) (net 35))
 (segment (start 103.932969 104.220031) (end 102.272999 105.880001) (width 0.25) (layer F.Cu) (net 35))
 (segment (start 102.272999 108.420001) (end 101.473 109.22) (width 0.25) (layer F.Cu) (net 37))
 (segment (start 106.193862 95.962691) (end 104.498956 97.657597) (width 0.25) (layer F.Cu) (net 37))
 (segment (start 104.498956 97.657597) (end 104.498956 106.194044) (width 0.25) (layer F.Cu) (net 37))
 (segment (start 104.498956 106.194044) (end 102.272999 108.420001) (width 0.25) (layer F.Cu) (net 37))
 (segment (start 102.272999 110.960001) (end 101.473 111.76) (width 0.25) (layer F.Cu) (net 39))
 (segment (start 104.948967 97.914694) (end 104.948967 108.284033) (width 0.25) (layer F.Cu) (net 39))
 (segment (start 106.547416 96.316245) (end 104.948967 97.914694) (width 0.25) (layer F.Cu) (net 39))
 (segment (start 104.948967 108.284033) (end 102.272999 110.960001) (width 0.25) (layer F.Cu) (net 39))
 (segment (start 102.272999 113.500001) (end 101.473 114.3) (width 0.25) (layer F.Cu) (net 41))
 (segment (start 105.398978 98.171789) (end 105.398978 110.374022) (width 0.25) (layer F.Cu) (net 41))
 (segment (start 106.900969 96.669798) (end 105.398978 98.171789) (width 0.25) (layer F.Cu) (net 41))
 (segment (start 105.398978 110.374022) (end 102.272999 113.500001) (width 0.25) (layer F.Cu) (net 41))
 (segment (start 105.848989 98.428884) (end 105.848989 112.464011) (width 0.25) (layer F.Cu) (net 43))
 (segment (start 107.254522 97.023351) (end 105.848989 98.428884) (width 0.25) (layer F.Cu) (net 43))
 (segment (start 105.848989 112.464011) (end 102.272999 116.040001) (width 0.25) (layer F.Cu) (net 43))
 (segment (start 102.272999 116.040001) (end 101.473 116.84) (width 0.25) (layer F.Cu) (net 43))
 (segment (start 107.608076 97.447599) (end 106.299 98.756675) (width 0.25) (layer F.Cu) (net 45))
 (segment (start 107.608076 97.376905) (end 107.608076 97.447599) (width 0.25) (layer F.Cu) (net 45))
 (segment (start 106.299 98.756675) (end 106.299 114.554) (width 0.25) (layer F.Cu) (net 45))
 (segment (start 106.299 114.554) (end 101.473 119.38) (width 0.25) (layer F.Cu) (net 45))
 (segment (start 107.961629 115.431371) (end 101.473 121.92) (width 0.25) (layer F.Cu) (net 47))
 (segment (start 107.961629 97.730458) (end 107.961629 115.431371) (width 0.25) (layer F.Cu) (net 47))
 (segment (start 110.224371 115.431371) (end 116.713 121.92) (width 0.25) (layer F.Cu) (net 2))
 (segment (start 110.224371 97.730458) (end 110.224371 115.431371) (width 0.25) (layer F.Cu) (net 2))
 (segment (start 111.887 98.685981) (end 111.108253 97.907234) (width 0.25) (layer F.Cu) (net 4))
 (segment (start 111.887 114.554) (end 111.887 98.685981) (width 0.25) (layer F.Cu) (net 4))
 (segment (start 111.108253 97.907234) (end 110.577924 97.376905) (width 0.25) (layer F.Cu) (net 4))
 (segment (start 116.713 119.38) (end 111.887 114.554) (width 0.25) (layer F.Cu) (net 4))
 (segment (start 112.337011 98.428884) (end 112.337011 112.464011) (width 0.25) (layer F.Cu) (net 6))
 (segment (start 110.931478 97.023351) (end 112.337011 98.428884) (width 0.25) (layer F.Cu) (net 6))
 (segment (start 112.337011 112.464011) (end 115.913001 116.040001) (width 0.25) (layer F.Cu) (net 6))
 (segment (start 115.913001 116.040001) (end 116.713 116.84) (width 0.25) (layer F.Cu) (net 6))
 (segment (start 112.903 98.287767) (end 111.285031 96.669798) (width 0.25) (layer F.Cu) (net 8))
 (segment (start 112.903 110.49) (end 112.903 98.287767) (width 0.25) (layer F.Cu) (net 8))
 (segment (start 116.713 114.3) (end 112.903 110.49) (width 0.25) (layer F.Cu) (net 8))
 (segment (start 115.913001 110.960001) (end 116.713 111.76) (width 0.25) (layer F.Cu) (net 10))
 (segment (start 113.353011 108.400011) (end 115.913001 110.960001) (width 0.25) (layer F.Cu) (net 10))
 (segment (start 111.638584 96.316245) (end 113.353011 98.030672) (width 0.25) (layer F.Cu) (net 10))
 (segment (start 113.353011 98.030672) (end 113.353011 108.400011) (width 0.25) (layer F.Cu) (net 10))
 (segment (start 113.803022 97.773575) (end 113.803022 106.310022) (width 0.25) (layer F.Cu) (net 12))
 (segment (start 113.803022 106.310022) (end 115.913001 108.420001) (width 0.25) (layer F.Cu) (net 12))
 (segment (start 115.913001 108.420001) (end 116.713 109.22) (width 0.25) (layer F.Cu) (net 12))
 (segment (start 111.992138 95.962691) (end 113.803022 97.773575) (width 0.25) (layer F.Cu) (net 12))
 (segment (start 112.345691 95.609138) (end 114.253033 97.51648) (width 0.25) (layer F.Cu) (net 14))
 (segment (start 115.913001 105.880001) (end 116.713 106.68) (width 0.25) (layer F.Cu) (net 14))
 (segment (start 114.253033 97.51648) (end 114.253033 104.220033) (width 0.25) (layer F.Cu) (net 14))
 (segment (start 114.253033 104.220033) (end 115.913001 105.880001) (width 0.25) (layer F.Cu) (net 14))
 (segment (start 113.229574 95.785913) (end 112.699245 95.255584) (width 0.25) (layer F.Cu) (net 16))
 (segment (start 116.713 104.14) (end 114.703044 102.130044) (width 0.25) (layer F.Cu) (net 16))
 (segment (start 114.703044 102.130044) (end 114.703044 97.259383) (width 0.25) (layer F.Cu) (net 16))
 (segment (start 114.703044 97.259383) (end 113.229574 95.785913) (width 0.25) (layer F.Cu) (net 16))
 (segment (start 113.583127 95.43236) (end 113.052798 94.902031) (width 0.25) (layer F.Cu) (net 18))
 (segment (start 115.153055 100.040055) (end 115.153055 97.002288) (width 0.25) (layer F.Cu) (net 18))
 (segment (start 115.153055 97.002288) (end 113.583127 95.43236) (width 0.25) (layer F.Cu) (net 18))
 (segment (start 116.713 101.6) (end 115.153055 100.040055) (width 0.25) (layer F.Cu) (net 18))
 (segment (start 115.603066 96.745193) (end 113.93668 95.078807) (width 0.25) (layer F.Cu) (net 20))
 (segment (start 115.603066 97.950066) (end 115.603066 96.745193) (width 0.25) (layer F.Cu) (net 20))
 (segment (start 113.93668 95.078807) (end 113.406351 94.548478) (width 0.25) (layer F.Cu) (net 20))
 (segment (start 116.713 99.06) (end 115.603066 97.950066) (width 0.25) (layer F.Cu) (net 20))
 (segment (start 116.084981 96.52) (end 116.713 96.52) (width 0.25) (layer F.Cu) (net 22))
 (segment (start 113.759905 94.194924) (end 116.084981 96.52) (width 0.25) (layer F.Cu) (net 22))
 (segment (start 116.574371 93.841371) (end 116.713 93.98) (width 0.25) (layer F.Cu) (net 24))
 (segment (start 114.113458 93.841371) (end 116.574371 93.841371) (width 0.25) (layer F.Cu) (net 24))
 (segment (start 116.574371 91.578629) (end 116.713 91.44) (width 0.25) (layer F.Cu) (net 26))
 (segment (start 114.113458 91.578629) (end 116.574371 91.578629) (width 0.25) (layer F.Cu) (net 26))
 (segment (start 116.084981 88.9) (end 116.713 88.9) (width 0.25) (layer F.Cu) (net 28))
 (segment (start 113.759905 91.225076) (end 116.084981 88.9) (width 0.25) (layer F.Cu) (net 28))
 (segment (start 115.545075 88.732798) (end 115.545075 87.527925) (width 0.25) (layer F.Cu) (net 30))
 (segment (start 115.913001 87.159999) (end 116.713 86.36) (width 0.25) (layer F.Cu) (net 30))
 (segment (start 113.406351 90.871522) (end 115.545075 88.732798) (width 0.25) (layer F.Cu) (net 30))
 (segment (start 115.545075 87.527925) (end 115.913001 87.159999) (width 0.25) (layer F.Cu) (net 30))
 (segment (start 115.913001 84.619999) (end 116.713 83.82) (width 0.25) (layer F.Cu) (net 32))
 (segment (start 115.095064 85.437936) (end 115.913001 84.619999) (width 0.25) (layer F.Cu) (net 32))
 (segment (start 113.052798 90.517969) (end 115.095064 88.475703) (width 0.25) (layer F.Cu) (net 32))
 (segment (start 115.095064 88.475703) (end 115.095064 85.437936) (width 0.25) (layer F.Cu) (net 32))
 (segment (start 112.699245 90.164416) (end 114.645053 88.218608) (width 0.25) (layer F.Cu) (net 34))
 (segment (start 115.913001 82.079999) (end 116.713 81.28) (width 0.25) (layer F.Cu) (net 34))
 (segment (start 114.645053 83.347947) (end 115.913001 82.079999) (width 0.25) (layer F.Cu) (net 34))
 (segment (start 114.645053 88.218608) (end 114.645053 83.347947) (width 0.25) (layer F.Cu) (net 34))
 (segment (start 114.137053 81.315947) (end 115.913001 79.539999) (width 0.25) (layer F.Cu) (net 36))
 (segment (start 115.913001 79.539999) (end 116.713 78.74) (width 0.25) (layer F.Cu) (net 36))
 (segment (start 114.137053 88.0195) (end 114.137053 81.315947) (width 0.25) (layer F.Cu) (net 36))
 (segment (start 112.345691 89.810862) (end 114.137053 88.0195) (width 0.25) (layer F.Cu) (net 36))
 (segment (start 115.913001 76.999999) (end 116.713 76.2) (width 0.25) (layer F.Cu) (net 38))
 (segment (start 113.687042 87.762405) (end 113.687042 79.225958) (width 0.25) (layer F.Cu) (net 38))
 (segment (start 113.687042 79.225958) (end 115.913001 76.999999) (width 0.25) (layer F.Cu) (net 38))
 (segment (start 111.992138 89.457309) (end 113.687042 87.762405) (width 0.25) (layer F.Cu) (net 38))
 (segment (start 113.237031 87.505308) (end 113.237031 77.135969) (width 0.25) (layer F.Cu) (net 40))
 (segment (start 111.638584 89.103755) (end 113.237031 87.505308) (width 0.25) (layer F.Cu) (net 40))
 (segment (start 115.913001 74.459999) (end 116.713 73.66) (width 0.25) (layer F.Cu) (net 40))
 (segment (start 113.237031 77.135969) (end 115.913001 74.459999) (width 0.25) (layer F.Cu) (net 40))
 (segment (start 111.285031 88.750202) (end 112.78702 87.248213) (width 0.25) (layer F.Cu) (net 42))
 (segment (start 112.78702 87.248213) (end 112.78702 75.04598) (width 0.25) (layer F.Cu) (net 42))
 (segment (start 112.78702 75.04598) (end 115.913001 71.919999) (width 0.25) (layer F.Cu) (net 42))
 (segment (start 115.913001 71.919999) (end 116.713 71.12) (width 0.25) (layer F.Cu) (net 42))
 (segment (start 115.913001 69.379999) (end 116.713 68.58) (width 0.25) (layer F.Cu) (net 44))
 (segment (start 112.20303 87.125097) (end 112.20303 73.08997) (width 0.25) (layer F.Cu) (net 44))
 (segment (start 112.20303 73.08997) (end 115.913001 69.379999) (width 0.25) (layer F.Cu) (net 44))
 (segment (start 110.931478 88.396649) (end 112.20303 87.125097) (width 0.25) (layer F.Cu) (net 44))
 (segment (start 115.913001 66.839999) (end 116.713 66.04) (width 0.25) (layer F.Cu) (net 46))
 (segment (start 111.753019 86.868) (end 111.753019 70.999981) (width 0.25) (layer F.Cu) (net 46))
 (segment (start 110.577924 88.043095) (end 111.753019 86.868) (width 0.25) (layer F.Cu) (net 46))
 (segment (start 111.753019 70.999981) (end 115.913001 66.839999) (width 0.25) (layer F.Cu) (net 46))
 (segment (start 110.224371 69.988629) (end 116.713 63.5) (width 0.25) (layer F.Cu) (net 48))
 (segment (start 110.224371 87.689542) (end 110.224371 69.988629) (width 0.25) (layer F.Cu) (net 48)))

